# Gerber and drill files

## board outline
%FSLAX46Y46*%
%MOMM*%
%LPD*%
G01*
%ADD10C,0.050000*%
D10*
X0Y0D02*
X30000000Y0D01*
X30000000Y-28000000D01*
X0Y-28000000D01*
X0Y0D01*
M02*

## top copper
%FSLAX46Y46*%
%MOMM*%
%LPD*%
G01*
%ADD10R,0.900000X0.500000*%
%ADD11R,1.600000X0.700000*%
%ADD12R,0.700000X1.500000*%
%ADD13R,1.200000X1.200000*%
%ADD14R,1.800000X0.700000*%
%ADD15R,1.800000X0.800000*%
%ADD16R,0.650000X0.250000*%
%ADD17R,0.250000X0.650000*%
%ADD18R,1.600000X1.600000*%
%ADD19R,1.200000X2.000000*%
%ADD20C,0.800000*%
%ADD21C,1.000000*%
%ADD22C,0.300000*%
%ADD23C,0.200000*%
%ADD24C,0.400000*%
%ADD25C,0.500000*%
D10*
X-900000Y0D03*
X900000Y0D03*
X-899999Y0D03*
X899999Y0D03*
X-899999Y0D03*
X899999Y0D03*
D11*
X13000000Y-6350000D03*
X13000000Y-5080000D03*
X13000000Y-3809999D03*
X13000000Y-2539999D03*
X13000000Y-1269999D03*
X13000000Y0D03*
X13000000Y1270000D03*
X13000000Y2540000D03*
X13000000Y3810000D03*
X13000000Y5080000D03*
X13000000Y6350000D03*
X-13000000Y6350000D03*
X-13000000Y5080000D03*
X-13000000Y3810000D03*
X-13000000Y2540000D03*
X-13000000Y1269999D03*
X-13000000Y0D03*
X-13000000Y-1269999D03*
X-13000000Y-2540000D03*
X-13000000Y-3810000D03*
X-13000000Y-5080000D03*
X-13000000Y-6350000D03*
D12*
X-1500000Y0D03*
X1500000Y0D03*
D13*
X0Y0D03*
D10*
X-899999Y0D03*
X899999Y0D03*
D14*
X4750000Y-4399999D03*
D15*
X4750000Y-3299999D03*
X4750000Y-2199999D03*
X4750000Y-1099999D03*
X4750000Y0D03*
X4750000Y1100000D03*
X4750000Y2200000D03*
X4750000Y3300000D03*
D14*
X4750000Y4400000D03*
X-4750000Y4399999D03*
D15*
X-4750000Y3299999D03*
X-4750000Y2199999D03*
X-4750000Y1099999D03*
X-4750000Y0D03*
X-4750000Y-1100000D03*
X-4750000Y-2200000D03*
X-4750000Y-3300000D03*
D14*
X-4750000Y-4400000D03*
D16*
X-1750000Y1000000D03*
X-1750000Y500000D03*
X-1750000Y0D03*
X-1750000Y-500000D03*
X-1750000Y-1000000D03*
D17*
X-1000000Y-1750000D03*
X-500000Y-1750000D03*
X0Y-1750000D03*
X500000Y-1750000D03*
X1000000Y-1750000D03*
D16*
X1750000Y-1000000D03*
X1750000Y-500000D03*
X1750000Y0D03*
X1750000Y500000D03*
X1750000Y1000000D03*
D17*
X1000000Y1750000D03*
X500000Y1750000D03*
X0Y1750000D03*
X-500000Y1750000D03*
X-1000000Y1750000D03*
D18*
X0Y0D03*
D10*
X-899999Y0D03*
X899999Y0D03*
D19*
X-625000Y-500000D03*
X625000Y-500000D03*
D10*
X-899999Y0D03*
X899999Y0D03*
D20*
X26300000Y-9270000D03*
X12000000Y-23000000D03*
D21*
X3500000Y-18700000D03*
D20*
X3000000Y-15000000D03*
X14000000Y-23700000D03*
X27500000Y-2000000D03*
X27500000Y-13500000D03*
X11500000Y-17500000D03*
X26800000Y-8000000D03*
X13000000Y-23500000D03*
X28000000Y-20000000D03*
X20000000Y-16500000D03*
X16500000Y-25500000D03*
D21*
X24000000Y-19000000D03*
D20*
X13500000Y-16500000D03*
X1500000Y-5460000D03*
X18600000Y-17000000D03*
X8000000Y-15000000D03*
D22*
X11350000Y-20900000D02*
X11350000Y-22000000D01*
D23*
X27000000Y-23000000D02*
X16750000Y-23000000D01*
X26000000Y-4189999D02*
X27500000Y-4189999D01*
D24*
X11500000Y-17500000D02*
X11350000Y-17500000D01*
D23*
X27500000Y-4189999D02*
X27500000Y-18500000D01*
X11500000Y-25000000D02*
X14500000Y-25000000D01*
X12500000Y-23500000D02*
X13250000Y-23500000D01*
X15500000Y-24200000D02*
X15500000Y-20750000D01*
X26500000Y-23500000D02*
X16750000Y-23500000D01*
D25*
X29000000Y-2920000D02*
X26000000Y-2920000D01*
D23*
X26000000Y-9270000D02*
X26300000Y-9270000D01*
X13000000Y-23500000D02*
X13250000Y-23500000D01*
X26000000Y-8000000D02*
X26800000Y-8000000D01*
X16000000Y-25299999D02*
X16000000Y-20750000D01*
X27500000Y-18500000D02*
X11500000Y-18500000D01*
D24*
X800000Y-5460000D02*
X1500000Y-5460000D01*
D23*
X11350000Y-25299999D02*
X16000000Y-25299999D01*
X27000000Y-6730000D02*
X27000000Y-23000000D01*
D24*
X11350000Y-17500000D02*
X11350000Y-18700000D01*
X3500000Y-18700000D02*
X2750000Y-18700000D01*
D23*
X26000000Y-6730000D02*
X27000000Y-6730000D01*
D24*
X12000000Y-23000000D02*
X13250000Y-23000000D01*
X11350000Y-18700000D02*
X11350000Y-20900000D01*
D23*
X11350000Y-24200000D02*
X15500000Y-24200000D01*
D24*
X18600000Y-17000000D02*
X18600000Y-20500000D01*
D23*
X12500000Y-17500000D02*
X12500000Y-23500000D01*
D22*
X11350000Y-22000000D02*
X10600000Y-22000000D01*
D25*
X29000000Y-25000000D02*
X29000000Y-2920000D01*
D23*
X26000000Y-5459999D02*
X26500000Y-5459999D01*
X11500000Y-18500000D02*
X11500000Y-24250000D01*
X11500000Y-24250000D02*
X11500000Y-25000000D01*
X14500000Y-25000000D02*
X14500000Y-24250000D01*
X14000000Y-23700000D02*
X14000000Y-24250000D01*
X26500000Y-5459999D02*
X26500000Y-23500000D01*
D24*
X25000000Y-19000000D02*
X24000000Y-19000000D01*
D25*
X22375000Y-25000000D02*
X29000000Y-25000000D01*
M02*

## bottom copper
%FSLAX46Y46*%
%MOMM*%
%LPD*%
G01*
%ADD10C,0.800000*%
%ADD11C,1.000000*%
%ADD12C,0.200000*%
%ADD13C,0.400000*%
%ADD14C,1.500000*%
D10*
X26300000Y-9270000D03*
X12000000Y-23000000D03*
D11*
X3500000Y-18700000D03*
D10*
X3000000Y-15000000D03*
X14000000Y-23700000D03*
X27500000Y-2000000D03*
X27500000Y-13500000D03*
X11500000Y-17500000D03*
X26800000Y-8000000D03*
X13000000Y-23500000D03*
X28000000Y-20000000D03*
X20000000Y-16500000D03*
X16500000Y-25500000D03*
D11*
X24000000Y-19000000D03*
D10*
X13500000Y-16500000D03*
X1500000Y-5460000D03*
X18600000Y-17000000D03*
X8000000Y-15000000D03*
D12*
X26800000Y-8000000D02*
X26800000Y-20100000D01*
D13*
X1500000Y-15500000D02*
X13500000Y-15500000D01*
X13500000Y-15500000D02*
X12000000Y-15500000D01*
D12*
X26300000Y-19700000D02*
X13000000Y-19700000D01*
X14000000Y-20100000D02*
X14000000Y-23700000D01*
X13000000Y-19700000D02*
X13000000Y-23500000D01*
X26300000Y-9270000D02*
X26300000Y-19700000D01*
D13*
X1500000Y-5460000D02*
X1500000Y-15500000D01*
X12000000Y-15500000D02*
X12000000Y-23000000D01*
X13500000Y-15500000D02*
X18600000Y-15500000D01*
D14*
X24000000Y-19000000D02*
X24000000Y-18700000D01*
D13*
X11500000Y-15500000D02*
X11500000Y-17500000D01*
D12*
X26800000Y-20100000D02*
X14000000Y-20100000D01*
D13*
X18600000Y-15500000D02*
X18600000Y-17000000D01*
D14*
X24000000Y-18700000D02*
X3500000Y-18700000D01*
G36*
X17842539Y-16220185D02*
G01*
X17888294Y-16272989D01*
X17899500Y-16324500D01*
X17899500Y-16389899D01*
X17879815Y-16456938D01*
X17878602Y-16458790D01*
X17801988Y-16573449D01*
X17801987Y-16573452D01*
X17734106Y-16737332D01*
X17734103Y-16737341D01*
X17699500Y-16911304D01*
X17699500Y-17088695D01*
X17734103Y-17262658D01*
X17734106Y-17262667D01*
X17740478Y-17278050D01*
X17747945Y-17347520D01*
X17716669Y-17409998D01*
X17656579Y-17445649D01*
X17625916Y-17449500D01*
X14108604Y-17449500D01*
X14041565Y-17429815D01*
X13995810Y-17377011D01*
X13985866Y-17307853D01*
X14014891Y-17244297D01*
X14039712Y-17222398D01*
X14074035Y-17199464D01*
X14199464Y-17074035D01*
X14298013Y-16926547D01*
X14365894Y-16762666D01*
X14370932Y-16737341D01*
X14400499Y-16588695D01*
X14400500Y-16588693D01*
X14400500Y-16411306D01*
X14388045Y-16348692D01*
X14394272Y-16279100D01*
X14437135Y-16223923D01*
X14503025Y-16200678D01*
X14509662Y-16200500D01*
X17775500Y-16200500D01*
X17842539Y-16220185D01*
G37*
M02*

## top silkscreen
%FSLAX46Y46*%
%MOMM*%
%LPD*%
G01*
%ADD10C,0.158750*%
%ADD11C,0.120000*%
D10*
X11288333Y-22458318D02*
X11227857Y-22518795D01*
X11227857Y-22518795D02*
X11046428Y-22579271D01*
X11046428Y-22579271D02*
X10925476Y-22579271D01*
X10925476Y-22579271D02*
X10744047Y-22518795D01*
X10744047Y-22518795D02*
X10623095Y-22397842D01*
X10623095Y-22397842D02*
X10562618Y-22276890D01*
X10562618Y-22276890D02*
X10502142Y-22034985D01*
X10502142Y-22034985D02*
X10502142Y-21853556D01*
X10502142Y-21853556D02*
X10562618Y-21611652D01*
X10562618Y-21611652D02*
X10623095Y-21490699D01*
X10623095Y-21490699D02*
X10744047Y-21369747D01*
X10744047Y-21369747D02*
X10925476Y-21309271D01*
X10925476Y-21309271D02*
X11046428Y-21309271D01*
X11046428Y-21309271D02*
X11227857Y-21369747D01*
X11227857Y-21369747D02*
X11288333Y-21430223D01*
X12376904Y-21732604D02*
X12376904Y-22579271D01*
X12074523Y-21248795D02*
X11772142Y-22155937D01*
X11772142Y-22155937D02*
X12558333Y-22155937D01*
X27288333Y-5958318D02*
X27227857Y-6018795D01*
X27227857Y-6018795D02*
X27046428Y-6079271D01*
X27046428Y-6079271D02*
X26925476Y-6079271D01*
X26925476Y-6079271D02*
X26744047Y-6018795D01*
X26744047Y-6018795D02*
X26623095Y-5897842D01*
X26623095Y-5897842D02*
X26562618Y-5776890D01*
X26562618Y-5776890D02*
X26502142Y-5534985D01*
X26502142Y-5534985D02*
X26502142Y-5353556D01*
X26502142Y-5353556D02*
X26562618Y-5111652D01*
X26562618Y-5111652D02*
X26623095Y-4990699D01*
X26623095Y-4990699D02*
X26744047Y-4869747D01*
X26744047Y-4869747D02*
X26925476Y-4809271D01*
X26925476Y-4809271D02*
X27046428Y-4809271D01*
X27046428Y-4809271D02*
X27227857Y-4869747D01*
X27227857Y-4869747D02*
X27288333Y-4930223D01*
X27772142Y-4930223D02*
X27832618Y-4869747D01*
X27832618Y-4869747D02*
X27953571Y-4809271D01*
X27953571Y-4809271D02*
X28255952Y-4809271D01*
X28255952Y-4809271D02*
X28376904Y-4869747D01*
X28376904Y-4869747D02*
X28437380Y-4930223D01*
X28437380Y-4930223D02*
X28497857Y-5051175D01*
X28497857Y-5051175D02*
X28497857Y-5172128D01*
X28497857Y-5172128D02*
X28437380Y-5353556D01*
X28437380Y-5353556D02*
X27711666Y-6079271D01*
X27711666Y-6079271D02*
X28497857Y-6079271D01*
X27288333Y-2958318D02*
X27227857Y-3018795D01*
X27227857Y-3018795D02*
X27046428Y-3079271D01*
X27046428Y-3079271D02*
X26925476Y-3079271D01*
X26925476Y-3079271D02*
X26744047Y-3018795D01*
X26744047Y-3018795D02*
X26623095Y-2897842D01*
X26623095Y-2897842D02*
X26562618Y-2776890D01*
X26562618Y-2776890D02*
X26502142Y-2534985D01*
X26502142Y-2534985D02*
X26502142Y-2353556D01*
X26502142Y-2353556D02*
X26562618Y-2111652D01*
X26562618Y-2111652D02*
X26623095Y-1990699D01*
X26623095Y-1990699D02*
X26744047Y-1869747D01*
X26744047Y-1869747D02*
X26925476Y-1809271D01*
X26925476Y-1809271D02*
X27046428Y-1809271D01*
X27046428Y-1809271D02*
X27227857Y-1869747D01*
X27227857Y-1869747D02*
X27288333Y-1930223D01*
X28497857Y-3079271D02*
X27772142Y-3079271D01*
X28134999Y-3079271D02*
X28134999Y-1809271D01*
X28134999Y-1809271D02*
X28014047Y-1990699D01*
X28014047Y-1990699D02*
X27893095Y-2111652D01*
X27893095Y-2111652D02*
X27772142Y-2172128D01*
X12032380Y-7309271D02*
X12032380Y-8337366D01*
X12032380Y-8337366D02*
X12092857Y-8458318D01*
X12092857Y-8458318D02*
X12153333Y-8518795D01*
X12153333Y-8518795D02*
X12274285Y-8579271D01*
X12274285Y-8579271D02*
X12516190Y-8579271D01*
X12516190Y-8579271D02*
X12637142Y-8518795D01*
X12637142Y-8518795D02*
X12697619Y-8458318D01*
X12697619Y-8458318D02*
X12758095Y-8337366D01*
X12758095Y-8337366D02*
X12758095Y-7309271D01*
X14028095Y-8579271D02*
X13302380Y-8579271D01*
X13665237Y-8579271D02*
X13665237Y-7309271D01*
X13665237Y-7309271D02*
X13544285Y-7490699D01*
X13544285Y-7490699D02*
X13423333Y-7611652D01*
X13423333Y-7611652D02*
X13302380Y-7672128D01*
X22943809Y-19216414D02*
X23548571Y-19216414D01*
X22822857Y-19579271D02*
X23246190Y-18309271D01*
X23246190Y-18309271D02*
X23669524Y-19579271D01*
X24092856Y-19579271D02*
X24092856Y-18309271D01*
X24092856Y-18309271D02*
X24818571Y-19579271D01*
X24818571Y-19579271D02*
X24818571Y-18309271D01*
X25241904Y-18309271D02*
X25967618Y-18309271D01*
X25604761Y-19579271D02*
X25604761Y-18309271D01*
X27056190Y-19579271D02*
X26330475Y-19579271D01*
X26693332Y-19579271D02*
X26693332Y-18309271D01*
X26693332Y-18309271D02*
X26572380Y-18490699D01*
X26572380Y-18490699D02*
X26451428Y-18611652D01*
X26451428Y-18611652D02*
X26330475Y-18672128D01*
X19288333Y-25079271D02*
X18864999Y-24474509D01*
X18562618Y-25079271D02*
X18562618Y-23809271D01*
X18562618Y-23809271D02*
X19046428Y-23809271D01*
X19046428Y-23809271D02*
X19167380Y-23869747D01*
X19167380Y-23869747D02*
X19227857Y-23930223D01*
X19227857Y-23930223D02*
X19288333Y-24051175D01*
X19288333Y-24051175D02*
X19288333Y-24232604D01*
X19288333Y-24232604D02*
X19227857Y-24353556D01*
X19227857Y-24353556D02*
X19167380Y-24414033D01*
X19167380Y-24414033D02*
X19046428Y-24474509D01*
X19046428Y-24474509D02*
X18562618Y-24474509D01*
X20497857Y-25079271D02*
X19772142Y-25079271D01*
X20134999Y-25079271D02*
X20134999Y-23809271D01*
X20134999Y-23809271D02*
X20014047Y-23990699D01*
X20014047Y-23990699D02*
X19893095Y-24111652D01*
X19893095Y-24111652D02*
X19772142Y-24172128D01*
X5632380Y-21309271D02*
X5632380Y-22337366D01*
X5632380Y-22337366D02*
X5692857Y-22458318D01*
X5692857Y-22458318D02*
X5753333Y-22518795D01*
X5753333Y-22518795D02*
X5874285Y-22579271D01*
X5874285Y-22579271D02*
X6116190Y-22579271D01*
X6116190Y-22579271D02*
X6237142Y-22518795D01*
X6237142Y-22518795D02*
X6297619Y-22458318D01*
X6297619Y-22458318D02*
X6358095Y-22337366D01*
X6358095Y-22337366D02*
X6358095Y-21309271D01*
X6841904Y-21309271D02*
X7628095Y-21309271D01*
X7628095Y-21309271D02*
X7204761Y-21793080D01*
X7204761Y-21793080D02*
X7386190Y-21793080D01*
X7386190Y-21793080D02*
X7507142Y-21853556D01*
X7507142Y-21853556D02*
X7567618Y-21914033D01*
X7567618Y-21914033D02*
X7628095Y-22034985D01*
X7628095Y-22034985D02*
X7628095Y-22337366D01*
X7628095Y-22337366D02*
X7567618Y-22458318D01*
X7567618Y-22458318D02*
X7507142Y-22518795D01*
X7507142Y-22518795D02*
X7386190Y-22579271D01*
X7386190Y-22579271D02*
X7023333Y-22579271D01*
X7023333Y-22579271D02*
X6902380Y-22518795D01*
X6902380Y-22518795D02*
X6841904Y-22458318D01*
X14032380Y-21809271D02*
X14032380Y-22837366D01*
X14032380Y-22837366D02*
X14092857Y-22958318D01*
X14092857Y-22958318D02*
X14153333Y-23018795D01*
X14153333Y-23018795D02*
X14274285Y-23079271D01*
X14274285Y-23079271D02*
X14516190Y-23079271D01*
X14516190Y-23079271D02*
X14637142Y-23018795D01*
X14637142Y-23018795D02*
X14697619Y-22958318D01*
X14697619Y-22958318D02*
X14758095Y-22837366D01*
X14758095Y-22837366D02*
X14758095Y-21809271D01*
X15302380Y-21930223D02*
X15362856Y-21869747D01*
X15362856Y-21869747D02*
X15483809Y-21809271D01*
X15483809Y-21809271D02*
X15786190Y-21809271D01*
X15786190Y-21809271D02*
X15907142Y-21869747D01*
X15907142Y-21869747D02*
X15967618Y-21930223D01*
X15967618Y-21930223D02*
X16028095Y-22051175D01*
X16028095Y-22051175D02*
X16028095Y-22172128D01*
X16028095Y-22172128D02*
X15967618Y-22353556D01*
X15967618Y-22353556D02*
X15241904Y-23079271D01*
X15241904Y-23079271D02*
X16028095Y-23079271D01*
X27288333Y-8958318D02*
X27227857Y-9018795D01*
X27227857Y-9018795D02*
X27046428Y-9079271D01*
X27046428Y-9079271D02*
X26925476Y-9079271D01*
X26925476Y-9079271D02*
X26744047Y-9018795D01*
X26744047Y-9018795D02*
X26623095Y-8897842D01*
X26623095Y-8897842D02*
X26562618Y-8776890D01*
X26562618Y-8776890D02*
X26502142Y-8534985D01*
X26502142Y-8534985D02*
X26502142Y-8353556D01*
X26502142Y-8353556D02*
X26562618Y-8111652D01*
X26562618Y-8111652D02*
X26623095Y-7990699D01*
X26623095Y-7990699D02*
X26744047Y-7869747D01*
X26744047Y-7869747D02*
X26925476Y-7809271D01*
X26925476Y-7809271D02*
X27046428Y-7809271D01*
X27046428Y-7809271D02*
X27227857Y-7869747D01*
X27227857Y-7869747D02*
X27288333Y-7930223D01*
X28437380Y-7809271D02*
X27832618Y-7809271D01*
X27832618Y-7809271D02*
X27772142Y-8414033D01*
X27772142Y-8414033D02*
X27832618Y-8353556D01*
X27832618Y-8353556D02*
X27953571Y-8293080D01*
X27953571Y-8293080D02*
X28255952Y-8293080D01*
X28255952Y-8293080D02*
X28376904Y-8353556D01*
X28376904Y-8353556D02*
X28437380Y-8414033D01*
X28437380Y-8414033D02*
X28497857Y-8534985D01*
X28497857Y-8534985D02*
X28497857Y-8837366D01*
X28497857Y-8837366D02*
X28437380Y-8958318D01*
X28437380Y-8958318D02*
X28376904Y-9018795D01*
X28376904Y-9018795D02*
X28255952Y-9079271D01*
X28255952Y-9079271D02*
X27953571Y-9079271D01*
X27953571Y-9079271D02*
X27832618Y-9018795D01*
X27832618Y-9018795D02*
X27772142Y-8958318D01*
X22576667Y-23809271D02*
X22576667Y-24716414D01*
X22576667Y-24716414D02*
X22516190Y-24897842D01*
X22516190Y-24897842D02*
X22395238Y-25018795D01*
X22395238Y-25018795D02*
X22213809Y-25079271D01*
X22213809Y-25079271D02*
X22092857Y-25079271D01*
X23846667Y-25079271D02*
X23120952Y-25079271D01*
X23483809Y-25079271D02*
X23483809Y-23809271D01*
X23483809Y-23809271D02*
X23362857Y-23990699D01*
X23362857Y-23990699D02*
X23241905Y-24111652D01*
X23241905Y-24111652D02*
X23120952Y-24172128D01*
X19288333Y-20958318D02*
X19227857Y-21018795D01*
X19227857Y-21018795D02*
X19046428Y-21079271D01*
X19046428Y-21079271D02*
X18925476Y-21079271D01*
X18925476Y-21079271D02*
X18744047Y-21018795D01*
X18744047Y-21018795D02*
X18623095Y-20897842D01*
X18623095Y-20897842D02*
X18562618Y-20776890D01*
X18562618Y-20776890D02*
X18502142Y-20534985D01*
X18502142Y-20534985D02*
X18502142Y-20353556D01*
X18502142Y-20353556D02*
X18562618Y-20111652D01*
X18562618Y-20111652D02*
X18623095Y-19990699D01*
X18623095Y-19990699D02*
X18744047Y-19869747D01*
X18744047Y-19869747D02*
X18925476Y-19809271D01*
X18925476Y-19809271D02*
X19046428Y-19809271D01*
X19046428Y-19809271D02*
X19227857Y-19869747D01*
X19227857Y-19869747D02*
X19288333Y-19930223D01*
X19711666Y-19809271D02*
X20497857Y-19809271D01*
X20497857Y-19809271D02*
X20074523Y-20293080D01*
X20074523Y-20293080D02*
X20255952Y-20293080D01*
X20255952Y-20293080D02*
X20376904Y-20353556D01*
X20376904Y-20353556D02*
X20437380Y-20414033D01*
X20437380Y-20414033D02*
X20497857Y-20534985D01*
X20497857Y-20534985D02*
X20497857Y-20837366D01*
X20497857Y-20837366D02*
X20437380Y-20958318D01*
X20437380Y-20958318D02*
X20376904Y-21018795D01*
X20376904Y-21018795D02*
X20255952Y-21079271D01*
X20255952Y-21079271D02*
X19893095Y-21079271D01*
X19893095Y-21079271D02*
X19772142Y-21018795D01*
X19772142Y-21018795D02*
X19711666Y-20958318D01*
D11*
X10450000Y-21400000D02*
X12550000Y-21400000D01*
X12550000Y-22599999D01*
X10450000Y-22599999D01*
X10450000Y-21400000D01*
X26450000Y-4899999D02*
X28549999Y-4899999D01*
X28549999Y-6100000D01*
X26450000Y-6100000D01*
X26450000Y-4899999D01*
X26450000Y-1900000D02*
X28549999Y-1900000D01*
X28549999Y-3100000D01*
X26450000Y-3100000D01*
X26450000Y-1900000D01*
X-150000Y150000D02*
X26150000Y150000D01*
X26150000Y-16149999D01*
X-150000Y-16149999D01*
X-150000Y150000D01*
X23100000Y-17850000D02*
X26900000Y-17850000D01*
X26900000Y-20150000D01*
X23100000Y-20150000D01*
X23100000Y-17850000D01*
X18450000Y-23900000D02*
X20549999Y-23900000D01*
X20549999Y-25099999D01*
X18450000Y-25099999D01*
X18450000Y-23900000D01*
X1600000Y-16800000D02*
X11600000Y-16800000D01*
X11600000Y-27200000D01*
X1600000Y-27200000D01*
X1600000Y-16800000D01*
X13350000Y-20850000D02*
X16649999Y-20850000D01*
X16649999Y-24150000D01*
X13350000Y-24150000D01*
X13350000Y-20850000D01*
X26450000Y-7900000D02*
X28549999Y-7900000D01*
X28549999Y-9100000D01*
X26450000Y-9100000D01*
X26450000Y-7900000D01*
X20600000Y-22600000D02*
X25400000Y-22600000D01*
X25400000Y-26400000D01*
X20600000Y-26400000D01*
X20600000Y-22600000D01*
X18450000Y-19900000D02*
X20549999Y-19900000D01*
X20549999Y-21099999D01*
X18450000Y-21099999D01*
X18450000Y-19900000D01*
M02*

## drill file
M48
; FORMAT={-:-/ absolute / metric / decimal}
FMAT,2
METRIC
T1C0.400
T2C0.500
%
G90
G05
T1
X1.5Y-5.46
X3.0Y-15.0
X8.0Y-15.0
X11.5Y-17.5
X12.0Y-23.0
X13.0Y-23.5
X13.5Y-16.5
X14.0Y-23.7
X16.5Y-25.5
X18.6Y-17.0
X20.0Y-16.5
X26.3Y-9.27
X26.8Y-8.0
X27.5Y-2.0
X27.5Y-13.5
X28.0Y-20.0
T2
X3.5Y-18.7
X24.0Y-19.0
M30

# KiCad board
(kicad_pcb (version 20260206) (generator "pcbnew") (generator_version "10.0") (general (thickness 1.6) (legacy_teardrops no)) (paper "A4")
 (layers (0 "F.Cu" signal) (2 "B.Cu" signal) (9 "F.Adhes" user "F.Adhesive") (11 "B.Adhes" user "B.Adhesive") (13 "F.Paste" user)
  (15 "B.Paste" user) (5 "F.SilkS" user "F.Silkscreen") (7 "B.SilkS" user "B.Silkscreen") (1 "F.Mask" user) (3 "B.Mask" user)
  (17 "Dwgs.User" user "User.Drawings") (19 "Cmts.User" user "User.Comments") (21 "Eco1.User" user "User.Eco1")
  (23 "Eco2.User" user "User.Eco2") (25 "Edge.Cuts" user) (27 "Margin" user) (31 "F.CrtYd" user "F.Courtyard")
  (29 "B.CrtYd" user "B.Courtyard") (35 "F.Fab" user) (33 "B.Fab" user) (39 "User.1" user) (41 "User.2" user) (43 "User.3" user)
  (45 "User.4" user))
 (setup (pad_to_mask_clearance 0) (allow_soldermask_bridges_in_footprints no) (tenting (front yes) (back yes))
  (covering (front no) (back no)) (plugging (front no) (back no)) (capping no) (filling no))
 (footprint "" (layer "F.Cu") (at 11.5 22)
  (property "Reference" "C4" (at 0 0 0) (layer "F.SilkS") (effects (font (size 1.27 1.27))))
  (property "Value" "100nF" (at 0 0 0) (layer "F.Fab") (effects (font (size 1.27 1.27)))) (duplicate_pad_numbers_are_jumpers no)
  (fp_rect (start -1.05 -0.6) (end 1.05 0.599999) (stroke (width 0.12) (type default)) (fill no) (layer "F.SilkS"))
  (pad "1" smd rect (at -12.4 -22) (size 0.9 0.5) (layers "F.Cu" "F.Mask" "F.Paste") (thermal_bridge_angle 45))
  (pad "2" smd rect (at -10.6 -22) (size 0.9 0.5) (layers "F.Cu" "F.Mask" "F.Paste") (thermal_bridge_angle 45)))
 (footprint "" (layer "F.Cu") (at 27.5 5.5)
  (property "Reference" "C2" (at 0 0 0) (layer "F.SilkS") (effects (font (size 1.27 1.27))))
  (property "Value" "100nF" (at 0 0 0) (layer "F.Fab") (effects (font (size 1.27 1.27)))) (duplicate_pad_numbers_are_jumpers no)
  (fp_rect (start -1.05 -0.600001) (end 1.049999 0.6) (stroke (width 0.12) (type default)) (fill no) (layer "F.SilkS"))
  (pad "1" smd rect (at -28.399999 -5.5) (size 0.9 0.5) (layers "F.Cu" "F.Mask" "F.Paste") (thermal_bridge_angle 45))
  (pad "2" smd rect (at -26.600001 -5.5) (size 0.9 0.5) (layers "F.Cu" "F.Mask" "F.Paste") (thermal_bridge_angle 45)))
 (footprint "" (layer "F.Cu") (at 27.5 2.5)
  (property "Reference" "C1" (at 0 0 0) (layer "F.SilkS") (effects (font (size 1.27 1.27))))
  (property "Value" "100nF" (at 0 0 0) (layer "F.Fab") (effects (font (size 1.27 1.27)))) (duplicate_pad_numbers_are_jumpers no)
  (fp_rect (start -1.05 -0.6) (end 1.049999 0.6) (stroke (width 0.12) (type default)) (fill no) (layer "F.SilkS"))
  (pad "1" smd rect (at -28.399999 -2.5) (size 0.9 0.5) (layers "F.Cu" "F.Mask" "F.Paste") (thermal_bridge_angle 45))
  (pad "2" smd rect (at -26.600001 -2.5) (size 0.9 0.5) (layers "F.Cu" "F.Mask" "F.Paste") (thermal_bridge_angle 45)))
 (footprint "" (layer "F.Cu") (at 13 8)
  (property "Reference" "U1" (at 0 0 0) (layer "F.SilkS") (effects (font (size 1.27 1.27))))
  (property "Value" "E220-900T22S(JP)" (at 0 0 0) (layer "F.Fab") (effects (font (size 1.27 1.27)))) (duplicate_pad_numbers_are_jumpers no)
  (fp_rect (start -13.15 -8.15) (end 13.15 8.149999) (stroke (width 0.12) (type default)) (fill no) (layer "F.SilkS"))
  (pad "1" smd rect (at 0 -1.65) (size 1.6 0.7) (layers "F.Cu" "F.Mask" "F.Paste") (thermal_bridge_angle 45))
  (pad "2" smd rect (at 0 -2.92) (size 1.6 0.7) (layers "F.Cu" "F.Mask" "F.Paste") (thermal_bridge_angle 45))
  (pad "3" smd rect (at 0 -4.190001) (size 1.6 0.7) (layers "F.Cu" "F.Mask" "F.Paste") (thermal_bridge_angle 45))
  (pad "4" smd rect (at 0 -5.460001) (size 1.6 0.7) (layers "F.Cu" "F.Mask" "F.Paste") (thermal_bridge_angle 45))
  (pad "5" smd rect (at 0 -6.730001) (size 1.6 0.7) (layers "F.Cu" "F.Mask" "F.Paste") (thermal_bridge_angle 45))
  (pad "6" smd rect (at 0 -8) (size 1.6 0.7) (layers "F.Cu" "F.Mask" "F.Paste") (thermal_bridge_angle 45))
  (pad "7" smd rect (at 0 -9.27) (size 1.6 0.7) (layers "F.Cu" "F.Mask" "F.Paste") (thermal_bridge_angle 45))
  (pad "8" smd rect (at 0 -10.54) (size 1.6 0.7) (layers "F.Cu" "F.Mask" "F.Paste") (thermal_bridge_angle 45))
  (pad "9" smd rect (at 0 -11.81) (size 1.6 0.7) (layers "F.Cu" "F.Mask" "F.Paste") (thermal_bridge_angle 45))
  (pad "10" smd rect (at 0 -13.08) (size 1.6 0.7) (layers "F.Cu" "F.Mask" "F.Paste") (thermal_bridge_angle 45))
  (pad "11" smd rect (at 0 -14.35) (size 1.6 0.7) (layers "F.Cu" "F.Mask" "F.Paste") (thermal_bridge_angle 45))
  (pad "12" smd rect (at -26 -14.35) (size 1.6 0.7) (layers "F.Cu" "F.Mask" "F.Paste") (thermal_bridge_angle 45))
  (pad "13" smd rect (at -26 -13.08) (size 1.6 0.7) (layers "F.Cu" "F.Mask" "F.Paste") (thermal_bridge_angle 45))
  (pad "14" smd rect (at -26 -11.81) (size 1.6 0.7) (layers "F.Cu" "F.Mask" "F.Paste") (thermal_bridge_angle 45))
  (pad "15" smd rect (at -26 -10.54) (size 1.6 0.7) (layers "F.Cu" "F.Mask" "F.Paste") (thermal_bridge_angle 45))
  (pad "16" smd rect (at -26 -9.269999) (size 1.6 0.7) (layers "F.Cu" "F.Mask" "F.Paste") (thermal_bridge_angle 45))
  (pad "17" smd rect (at -26 -8) (size 1.6 0.7) (layers "F.Cu" "F.Mask" "F.Paste") (thermal_bridge_angle 45))
  (pad "18" smd rect (at -26 -6.730001) (size 1.6 0.7) (layers "F.Cu" "F.Mask" "F.Paste") (thermal_bridge_angle 45))
  (pad "19" smd rect (at -26 -5.46) (size 1.6 0.7) (layers "F.Cu" "F.Mask" "F.Paste") (thermal_bridge_angle 45))
  (pad "20" smd rect (at -26 -4.19) (size 1.6 0.7) (layers "F.Cu" "F.Mask" "F.Paste") (thermal_bridge_angle 45))
  (pad "21" smd rect (at -26 -2.92) (size 1.6 0.7) (layers "F.Cu" "F.Mask" "F.Paste") (thermal_bridge_angle 45))
  (pad "22" smd rect (at -26 -1.65) (size 1.6 0.7) (layers "F.Cu" "F.Mask" "F.Paste") (thermal_bridge_angle 45)))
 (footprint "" (layer "F.Cu") (at 25 19)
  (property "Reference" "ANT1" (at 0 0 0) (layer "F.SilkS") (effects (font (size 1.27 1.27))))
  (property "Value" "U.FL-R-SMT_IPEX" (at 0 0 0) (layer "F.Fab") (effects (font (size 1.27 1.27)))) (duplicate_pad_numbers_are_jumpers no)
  (fp_rect (start -1.9 -1.15) (end 1.9 1.15) (stroke (width 0.12) (type default)) (fill no) (layer "F.SilkS"))
  (pad "G1" smd rect (at -26.5 -19) (size 0.7 1.5) (layers "F.Cu" "F.Mask" "F.Paste") (thermal_bridge_angle 45))
  (pad "G2" smd rect (at -23.5 -19) (size 0.7 1.5) (layers "F.Cu" "F.Mask" "F.Paste") (thermal_bridge_angle 45))
  (pad "S" smd rect (at -25 -19) (size 1.2 1.2) (layers "F.Cu" "F.Mask" "F.Paste") (thermal_bridge_angle 45)))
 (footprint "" (layer "F.Cu") (at 19.5 24.5)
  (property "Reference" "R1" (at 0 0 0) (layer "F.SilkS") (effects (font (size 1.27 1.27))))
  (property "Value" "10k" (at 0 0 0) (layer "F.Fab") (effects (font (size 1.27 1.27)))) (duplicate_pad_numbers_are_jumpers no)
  (fp_rect (start -1.05 -0.6) (end 1.049999 0.599999) (stroke (width 0.12) (type default)) (fill no) (layer "F.SilkS"))
  (pad "1" smd rect (at -20.399999 -24.5) (size 0.9 0.5) (layers "F.Cu" "F.Mask" "F.Paste") (thermal_bridge_angle 45))
  (pad "2" smd rect (at -18.600001 -24.5) (size 0.9 0.5) (layers "F.Cu" "F.Mask" "F.Paste") (thermal_bridge_angle 45)))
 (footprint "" (layer "F.Cu") (at 6.6 22)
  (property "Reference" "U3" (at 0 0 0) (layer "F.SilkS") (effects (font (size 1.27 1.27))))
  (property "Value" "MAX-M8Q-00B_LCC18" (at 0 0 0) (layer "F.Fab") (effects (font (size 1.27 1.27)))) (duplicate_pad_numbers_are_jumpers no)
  (fp_rect (start -5 -5.2) (end 5 5.2) (stroke (width 0.12) (type default)) (fill no) (layer "F.SilkS"))
  (pad "1" smd rect (at -1.85 -17.600001) (size 1.8 0.7) (layers "F.Cu" "F.Mask" "F.Paste") (thermal_bridge_angle 45))
  (pad "2" smd rect (at -1.85 -18.700001) (size 1.8 0.8) (layers "F.Cu" "F.Mask" "F.Paste") (thermal_bridge_angle 45))
  (pad "3" smd rect (at -1.85 -19.800001) (size 1.8 0.8) (layers "F.Cu" "F.Mask" "F.Paste") (thermal_bridge_angle 45))
  (pad "4" smd rect (at -1.85 -20.900001) (size 1.8 0.8) (layers "F.Cu" "F.Mask" "F.Paste") (thermal_bridge_angle 45))
  (pad "5" smd rect (at -1.85 -22) (size 1.8 0.8) (layers "F.Cu" "F.Mask" "F.Paste") (thermal_bridge_angle 45))
  (pad "6" smd rect (at -1.85 -23.1) (size 1.8 0.8) (layers "F.Cu" "F.Mask" "F.Paste") (thermal_bridge_angle 45))
  (pad "7" smd rect (at -1.85 -24.2) (size 1.8 0.8) (layers "F.Cu" "F.Mask" "F.Paste") (thermal_bridge_angle 45))
  (pad "8" smd rect (at -1.85 -25.3) (size 1.8 0.8) (layers "F.Cu" "F.Mask" "F.Paste") (thermal_bridge_angle 45))
  (pad "9" smd rect (at -1.85 -26.4) (size 1.8 0.7) (layers "F.Cu" "F.Mask" "F.Paste") (thermal_bridge_angle 45))
  (pad "10" smd rect (at -11.35 -26.399999) (size 1.8 0.7) (layers "F.Cu" "F.Mask" "F.Paste") (thermal_bridge_angle 45))
  (pad "11" smd rect (at -11.35 -25.299999) (size 1.8 0.8) (layers "F.Cu" "F.Mask" "F.Paste") (thermal_bridge_angle 45))
  (pad "12" smd rect (at -11.35 -24.199999) (size 1.8 0.8) (layers "F.Cu" "F.Mask" "F.Paste") (thermal_bridge_angle 45))
  (pad "13" smd rect (at -11.35 -23.099999) (size 1.8 0.8) (layers "F.Cu" "F.Mask" "F.Paste") (thermal_bridge_angle 45))
  (pad "14" smd rect (at -11.35 -22) (size 1.8 0.8) (layers "F.Cu" "F.Mask" "F.Paste") (thermal_bridge_angle 45))
  (pad "15" smd rect (at -11.35 -20.9) (size 1.8 0.8) (layers "F.Cu" "F.Mask" "F.Paste") (thermal_bridge_angle 45))
  (pad "16" smd rect (at -11.35 -19.8) (size 1.8 0.8) (layers "F.Cu" "F.Mask" "F.Paste") (thermal_bridge_angle 45))
  (pad "17" smd rect (at -11.35 -18.7) (size 1.8 0.8) (layers "F.Cu" "F.Mask" "F.Paste") (thermal_bridge_angle 45))
  (pad "18" smd rect (at -11.35 -17.6) (size 1.8 0.7) (layers "F.Cu" "F.Mask" "F.Paste") (thermal_bridge_angle 45)))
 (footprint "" (layer "F.Cu") (at 15 22.5)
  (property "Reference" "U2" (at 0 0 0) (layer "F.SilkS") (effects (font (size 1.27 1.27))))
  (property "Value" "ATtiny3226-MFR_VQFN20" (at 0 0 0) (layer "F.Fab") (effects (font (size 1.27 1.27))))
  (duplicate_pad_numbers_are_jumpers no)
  (fp_rect (start -1.65 -1.65) (end 1.649999 1.65) (stroke (width 0.12) (type default)) (fill no) (layer "F.SilkS"))
  (pad "1" smd rect (at -16.75 -23.5) (size 0.65 0.25) (layers "F.Cu" "F.Mask" "F.Paste") (thermal_bridge_angle 45))
  (pad "2" smd rect (at -16.75 -23) (size 0.65 0.25) (layers "F.Cu" "F.Mask" "F.Paste") (thermal_bridge_angle 45))
  (pad "3" smd rect (at -16.75 -22.5) (size 0.65 0.25) (layers "F.Cu" "F.Mask" "F.Paste") (thermal_bridge_angle 45))
  (pad "4" smd rect (at -16.75 -22) (size 0.65 0.25) (layers "F.Cu" "F.Mask" "F.Paste") (thermal_bridge_angle 45))
  (pad "5" smd rect (at -16.75 -21.5) (size 0.65 0.25) (layers "F.Cu" "F.Mask" "F.Paste") (thermal_bridge_angle 45))
  (pad "6" smd rect (at -16 -20.75) (size 0.25 0.65) (layers "F.Cu" "F.Mask" "F.Paste") (thermal_bridge_angle 45))
  (pad "7" smd rect (at -15.5 -20.75) (size 0.25 0.65) (layers "F.Cu" "F.Mask" "F.Paste") (thermal_bridge_angle 45))
  (pad "8" smd rect (at -15 -20.75) (size 0.25 0.65) (layers "F.Cu" "F.Mask" "F.Paste") (thermal_bridge_angle 45))
  (pad "9" smd rect (at -14.5 -20.75) (size 0.25 0.65) (layers "F.Cu" "F.Mask" "F.Paste") (thermal_bridge_angle 45))
  (pad "10" smd rect (at -14 -20.75) (size 0.25 0.65) (layers "F.Cu" "F.Mask" "F.Paste") (thermal_bridge_angle 45))
  (pad "11" smd rect (at -13.25 -21.5) (size 0.65 0.25) (layers "F.Cu" "F.Mask" "F.Paste") (thermal_bridge_angle 45))
  (pad "12" smd rect (at -13.25 -22) (size 0.65 0.25) (layers "F.Cu" "F.Mask" "F.Paste") (thermal_bridge_angle 45))
  (pad "13" smd rect (at -13.25 -22.5) (size 0.65 0.25) (layers "F.Cu" "F.Mask" "F.Paste") (thermal_bridge_angle 45))
  (pad "14" smd rect (at -13.25 -23) (size 0.65 0.25) (layers "F.Cu" "F.Mask" "F.Paste") (thermal_bridge_angle 45))
  (pad "15" smd rect (at -13.25 -23.5) (size 0.65 0.25) (layers "F.Cu" "F.Mask" "F.Paste") (thermal_bridge_angle 45))
  (pad "16" smd rect (at -14 -24.25) (size 0.25 0.65) (layers "F.Cu" "F.Mask" "F.Paste") (thermal_bridge_angle 45))
  (pad "17" smd rect (at -14.5 -24.25) (size 0.25 0.65) (layers "F.Cu" "F.Mask" "F.Paste") (thermal_bridge_angle 45))
  (pad "18" smd rect (at -15 -24.25) (size 0.25 0.65) (layers "F.Cu" "F.Mask" "F.Paste") (thermal_bridge_angle 45))
  (pad "19" smd rect (at -15.5 -24.25) (size 0.25 0.65) (layers "F.Cu" "F.Mask" "F.Paste") (thermal_bridge_angle 45))
  (pad "20" smd rect (at -16 -24.25) (size 0.25 0.65) (layers "F.Cu" "F.Mask" "F.Paste") (thermal_bridge_angle 45))
  (pad "EP" smd rect (at -15 -22.5) (size 1.6 1.6) (layers "F.Cu" "F.Mask" "F.Paste") (thermal_bridge_angle 45)))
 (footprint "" (layer "F.Cu") (at 27.5 8.5)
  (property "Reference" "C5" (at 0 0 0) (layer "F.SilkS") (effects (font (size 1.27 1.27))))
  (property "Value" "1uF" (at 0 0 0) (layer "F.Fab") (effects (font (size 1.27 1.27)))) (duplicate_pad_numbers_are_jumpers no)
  (fp_rect (start -1.05 -0.6) (end 1.049999 0.6) (stroke (width 0.12) (type default)) (fill no) (layer "F.SilkS"))
  (pad "1" smd rect (at -28.399999 -8.5) (size 0.9 0.5) (layers "F.Cu" "F.Mask" "F.Paste") (thermal_bridge_angle 45))
  (pad "2" smd rect (at -26.600001 -8.5) (size 0.9 0.5) (layers "F.Cu" "F.Mask" "F.Paste") (thermal_bridge_angle 45)))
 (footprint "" (layer "F.Cu") (at 23 24.5)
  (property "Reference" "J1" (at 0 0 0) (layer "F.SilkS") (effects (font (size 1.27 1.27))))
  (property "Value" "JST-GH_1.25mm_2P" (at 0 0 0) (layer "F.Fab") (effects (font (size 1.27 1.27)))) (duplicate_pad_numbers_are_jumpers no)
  (fp_rect (start -2.4 -1.9) (end 2.4 1.9) (stroke (width 0.12) (type default)) (fill no) (layer "F.SilkS"))
  (pad "1" smd rect (at -23.625 -24) (size 1.2 2) (layers "F.Cu" "F.Mask" "F.Paste") (thermal_bridge_angle 45))
  (pad "2" smd rect (at -22.375 -24) (size 1.2 2) (layers "F.Cu" "F.Mask" "F.Paste") (thermal_bridge_angle 45)))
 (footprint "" (layer "F.Cu") (at 19.5 20.5)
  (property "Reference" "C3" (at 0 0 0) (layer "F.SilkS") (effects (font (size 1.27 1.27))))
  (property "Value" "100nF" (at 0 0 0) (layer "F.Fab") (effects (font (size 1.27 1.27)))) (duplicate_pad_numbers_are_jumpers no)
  (fp_rect (start -1.05 -0.6) (end 1.049999 0.599999) (stroke (width 0.12) (type default)) (fill no) (layer "F.SilkS"))
  (pad "1" smd rect (at -20.399999 -20.5) (size 0.9 0.5) (layers "F.Cu" "F.Mask" "F.Paste") (thermal_bridge_angle 45))
  (pad "2" smd rect (at -18.600001 -20.5) (size 0.9 0.5) (layers "F.Cu" "F.Mask" "F.Paste") (thermal_bridge_angle 45)))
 (gr_rect (start 0 0) (end 30 28) (stroke (width 0.05) (type default)) (fill no) (layer "Edge.Cuts"))
 (segment (start 11.35 20.9) (end 11.35 22) (width 0.3) (layer "F.Cu") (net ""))
 (segment (start 27 23) (end 16.75 23) (width 0.2) (layer "F.Cu") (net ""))
 (segment (start 26 4.189999) (end 27.5 4.189999) (width 0.2) (layer "F.Cu") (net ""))
 (segment (start 11.5 17.5) (end 11.35 17.5) (width 0.4) (layer "F.Cu") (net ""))
 (segment (start 27.5 4.189999) (end 27.5 18.5) (width 0.2) (layer "F.Cu") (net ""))
 (segment (start 11.5 25) (end 14.5 25) (width 0.2) (layer "F.Cu") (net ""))
 (segment (start 12.5 23.5) (end 13.25 23.5) (width 0.2) (layer "F.Cu") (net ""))
 (segment (start 15.5 24.2) (end 15.5 20.75) (width 0.2) (layer "F.Cu") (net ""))
 (segment (start 26.5 23.5) (end 16.75 23.5) (width 0.2) (layer "F.Cu") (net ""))
 (segment (start 29 2.92) (end 26 2.92) (width 0.5) (layer "F.Cu") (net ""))
 (segment (start 26 9.27) (end 26.3 9.27) (width 0.2) (layer "F.Cu") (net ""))
 (segment (start 13 23.5) (end 13.25 23.5) (width 0.2) (layer "F.Cu") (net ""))
 (segment (start 26 8) (end 26.8 8) (width 0.2) (layer "F.Cu") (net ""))
 (segment (start 16 25.299999) (end 16 20.75) (width 0.2) (layer "F.Cu") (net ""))
 (segment (start 27.5 18.5) (end 11.5 18.5) (width 0.2) (layer "F.Cu") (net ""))
 (segment (start 0.8 5.46) (end 1.5 5.46) (width 0.4) (layer "F.Cu") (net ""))
 (segment (start 11.35 25.299999) (end 16 25.299999) (width 0.2) (layer "F.Cu") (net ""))
 (segment (start 27 6.73) (end 27 23) (width 0.2) (layer "F.Cu") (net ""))
 (segment (start 11.35 17.5) (end 11.35 18.7) (width 0.4) (layer "F.Cu") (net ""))
 (segment (start 3.5 18.7) (end 2.75 18.7) (width 0.4) (layer "F.Cu") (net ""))
 (segment (start 26 6.73) (end 27 6.73) (width 0.2) (layer "F.Cu") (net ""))
 (segment (start 12 23) (end 13.25 23) (width 0.4) (layer "F.Cu") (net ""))
 (segment (start 11.35 18.7) (end 11.35 20.9) (width 0.4) (layer "F.Cu") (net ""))
 (segment (start 11.35 24.2) (end 15.5 24.2) (width 0.2) (layer "F.Cu") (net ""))
 (segment (start 18.6 17) (end 18.6 20.5) (width 0.4) (layer "F.Cu") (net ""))
 (segment (start 12.5 17.5) (end 12.5 23.5) (width 0.2) (layer "F.Cu") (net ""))
 (segment (start 11.35 22) (end 10.6 22) (width 0.3) (layer "F.Cu") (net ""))
 (segment (start 29 25) (end 29 2.92) (width 0.5) (layer "F.Cu") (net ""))
 (segment (start 26 5.459999) (end 26.5 5.459999) (width 0.2) (layer "F.Cu") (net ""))
 (segment (start 11.5 18.5) (end 11.5 24.25) (width 0.2) (layer "F.Cu") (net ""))
 (segment (start 11.5 24.25) (end 11.5 25) (width 0.2) (layer "F.Cu") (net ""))
 (segment (start 14.5 25) (end 14.5 24.25) (width 0.2) (layer "F.Cu") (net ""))
 (segment (start 14 23.7) (end 14 24.25) (width 0.2) (layer "F.Cu") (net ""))
 (segment (start 26.5 5.459999) (end 26.5 23.5) (width 0.2) (layer "F.Cu") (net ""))
 (segment (start 25 19) (end 24 19) (width 0.4) (layer "F.Cu") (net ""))
 (segment (start 22.375 25) (end 29 25) (width 0.5) (layer "F.Cu") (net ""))
 (via (at 26.3 9.27) (size 0.8) (drill 0.4) (layers "F.Cu" "B.Cu") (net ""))
 (via (at 12 23) (size 0.8) (drill 0.4) (layers "F.Cu" "B.Cu") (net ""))
 (via (at 3.5 18.7) (size 1) (drill 0.5) (layers "F.Cu" "B.Cu") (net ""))
 (via (at 3 15) (size 0.8) (drill 0.4) (layers "F.Cu" "B.Cu") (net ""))
 (via (at 14 23.7) (size 0.8) (drill 0.4) (layers "F.Cu" "B.Cu") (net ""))
 (via (at 27.5 2) (size 0.8) (drill 0.4) (layers "F.Cu" "B.Cu") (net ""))
 (via (at 27.5 13.5) (size 0.8) (drill 0.4) (layers "F.Cu" "B.Cu") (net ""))
 (via (at 11.5 17.5) (size 0.8) (drill 0.4) (layers "F.Cu" "B.Cu") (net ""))
 (via (at 26.8 8) (size 0.8) (drill 0.4) (layers "F.Cu" "B.Cu") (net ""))
 (via (at 13 23.5) (size 0.8) (drill 0.4) (layers "F.Cu" "B.Cu") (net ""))
 (via (at 28 20) (size 0.8) (drill 0.4) (layers "F.Cu" "B.Cu") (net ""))
 (via (at 20 16.5) (size 0.8) (drill 0.4) (layers "F.Cu" "B.Cu") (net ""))
 (via (at 16.5 25.5) (size 0.8) (drill 0.4) (layers "F.Cu" "B.Cu") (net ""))
 (via (at 24 19) (size 1) (drill 0.5) (layers "F.Cu" "B.Cu") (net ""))
 (via (at 13.5 16.5) (size 0.8) (drill 0.4) (layers "F.Cu" "B.Cu") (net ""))
 (via (at 1.5 5.46) (size 0.8) (drill 0.4) (layers "F.Cu" "B.Cu") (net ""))
 (via (at 18.6 17) (size 0.8) (drill 0.4) (layers "F.Cu" "B.Cu") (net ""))
 (via (at 8 15) (size 0.8) (drill 0.4) (layers "F.Cu" "B.Cu") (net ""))
 (segment (start 26.8 8) (end 26.8 20.1) (width 0.2) (layer "B.Cu") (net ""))
 (segment (start 1.5 15.5) (end 13.5 15.5) (width 0.4) (layer "B.Cu") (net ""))
 (segment (start 13.5 15.5) (end 12 15.5) (width 0.4) (layer "B.Cu") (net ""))
 (segment (start 26.3 19.7) (end 13 19.7) (width 0.2) (layer "B.Cu") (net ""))
 (segment (start 14 20.1) (end 14 23.7) (width 0.2) (layer "B.Cu") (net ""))
 (segment (start 13 19.7) (end 13 23.5) (width 0.2) (layer "B.Cu") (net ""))
 (segment (start 26.3 9.27) (end 26.3 19.7) (width 0.2) (layer "B.Cu") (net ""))
 (segment (start 1.5 5.46) (end 1.5 15.5) (width 0.4) (layer "B.Cu") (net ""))
 (segment (start 12 15.5) (end 12 23) (width 0.4) (layer "B.Cu") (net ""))
 (segment (start 13.5 15.5) (end 18.6 15.5) (width 0.4) (layer "B.Cu") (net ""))
 (segment (start 24 19) (end 24 18.7) (width 1.5) (layer "B.Cu") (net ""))
 (segment (start 11.5 15.5) (end 11.5 17.5) (width 0.4) (layer "B.Cu") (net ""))
 (segment (start 26.8 20.1) (end 14 20.1) (width 0.2) (layer "B.Cu") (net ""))
 (segment (start 18.6 15.5) (end 18.6 17) (width 0.4) (layer "B.Cu") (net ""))
 (segment (start 24 18.7) (end 3.5 18.7) (width 1.5) (layer "B.Cu") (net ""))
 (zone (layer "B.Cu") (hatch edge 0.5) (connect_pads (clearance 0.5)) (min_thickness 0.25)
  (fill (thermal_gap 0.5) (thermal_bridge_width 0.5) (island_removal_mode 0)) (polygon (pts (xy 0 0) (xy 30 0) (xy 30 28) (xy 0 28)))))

